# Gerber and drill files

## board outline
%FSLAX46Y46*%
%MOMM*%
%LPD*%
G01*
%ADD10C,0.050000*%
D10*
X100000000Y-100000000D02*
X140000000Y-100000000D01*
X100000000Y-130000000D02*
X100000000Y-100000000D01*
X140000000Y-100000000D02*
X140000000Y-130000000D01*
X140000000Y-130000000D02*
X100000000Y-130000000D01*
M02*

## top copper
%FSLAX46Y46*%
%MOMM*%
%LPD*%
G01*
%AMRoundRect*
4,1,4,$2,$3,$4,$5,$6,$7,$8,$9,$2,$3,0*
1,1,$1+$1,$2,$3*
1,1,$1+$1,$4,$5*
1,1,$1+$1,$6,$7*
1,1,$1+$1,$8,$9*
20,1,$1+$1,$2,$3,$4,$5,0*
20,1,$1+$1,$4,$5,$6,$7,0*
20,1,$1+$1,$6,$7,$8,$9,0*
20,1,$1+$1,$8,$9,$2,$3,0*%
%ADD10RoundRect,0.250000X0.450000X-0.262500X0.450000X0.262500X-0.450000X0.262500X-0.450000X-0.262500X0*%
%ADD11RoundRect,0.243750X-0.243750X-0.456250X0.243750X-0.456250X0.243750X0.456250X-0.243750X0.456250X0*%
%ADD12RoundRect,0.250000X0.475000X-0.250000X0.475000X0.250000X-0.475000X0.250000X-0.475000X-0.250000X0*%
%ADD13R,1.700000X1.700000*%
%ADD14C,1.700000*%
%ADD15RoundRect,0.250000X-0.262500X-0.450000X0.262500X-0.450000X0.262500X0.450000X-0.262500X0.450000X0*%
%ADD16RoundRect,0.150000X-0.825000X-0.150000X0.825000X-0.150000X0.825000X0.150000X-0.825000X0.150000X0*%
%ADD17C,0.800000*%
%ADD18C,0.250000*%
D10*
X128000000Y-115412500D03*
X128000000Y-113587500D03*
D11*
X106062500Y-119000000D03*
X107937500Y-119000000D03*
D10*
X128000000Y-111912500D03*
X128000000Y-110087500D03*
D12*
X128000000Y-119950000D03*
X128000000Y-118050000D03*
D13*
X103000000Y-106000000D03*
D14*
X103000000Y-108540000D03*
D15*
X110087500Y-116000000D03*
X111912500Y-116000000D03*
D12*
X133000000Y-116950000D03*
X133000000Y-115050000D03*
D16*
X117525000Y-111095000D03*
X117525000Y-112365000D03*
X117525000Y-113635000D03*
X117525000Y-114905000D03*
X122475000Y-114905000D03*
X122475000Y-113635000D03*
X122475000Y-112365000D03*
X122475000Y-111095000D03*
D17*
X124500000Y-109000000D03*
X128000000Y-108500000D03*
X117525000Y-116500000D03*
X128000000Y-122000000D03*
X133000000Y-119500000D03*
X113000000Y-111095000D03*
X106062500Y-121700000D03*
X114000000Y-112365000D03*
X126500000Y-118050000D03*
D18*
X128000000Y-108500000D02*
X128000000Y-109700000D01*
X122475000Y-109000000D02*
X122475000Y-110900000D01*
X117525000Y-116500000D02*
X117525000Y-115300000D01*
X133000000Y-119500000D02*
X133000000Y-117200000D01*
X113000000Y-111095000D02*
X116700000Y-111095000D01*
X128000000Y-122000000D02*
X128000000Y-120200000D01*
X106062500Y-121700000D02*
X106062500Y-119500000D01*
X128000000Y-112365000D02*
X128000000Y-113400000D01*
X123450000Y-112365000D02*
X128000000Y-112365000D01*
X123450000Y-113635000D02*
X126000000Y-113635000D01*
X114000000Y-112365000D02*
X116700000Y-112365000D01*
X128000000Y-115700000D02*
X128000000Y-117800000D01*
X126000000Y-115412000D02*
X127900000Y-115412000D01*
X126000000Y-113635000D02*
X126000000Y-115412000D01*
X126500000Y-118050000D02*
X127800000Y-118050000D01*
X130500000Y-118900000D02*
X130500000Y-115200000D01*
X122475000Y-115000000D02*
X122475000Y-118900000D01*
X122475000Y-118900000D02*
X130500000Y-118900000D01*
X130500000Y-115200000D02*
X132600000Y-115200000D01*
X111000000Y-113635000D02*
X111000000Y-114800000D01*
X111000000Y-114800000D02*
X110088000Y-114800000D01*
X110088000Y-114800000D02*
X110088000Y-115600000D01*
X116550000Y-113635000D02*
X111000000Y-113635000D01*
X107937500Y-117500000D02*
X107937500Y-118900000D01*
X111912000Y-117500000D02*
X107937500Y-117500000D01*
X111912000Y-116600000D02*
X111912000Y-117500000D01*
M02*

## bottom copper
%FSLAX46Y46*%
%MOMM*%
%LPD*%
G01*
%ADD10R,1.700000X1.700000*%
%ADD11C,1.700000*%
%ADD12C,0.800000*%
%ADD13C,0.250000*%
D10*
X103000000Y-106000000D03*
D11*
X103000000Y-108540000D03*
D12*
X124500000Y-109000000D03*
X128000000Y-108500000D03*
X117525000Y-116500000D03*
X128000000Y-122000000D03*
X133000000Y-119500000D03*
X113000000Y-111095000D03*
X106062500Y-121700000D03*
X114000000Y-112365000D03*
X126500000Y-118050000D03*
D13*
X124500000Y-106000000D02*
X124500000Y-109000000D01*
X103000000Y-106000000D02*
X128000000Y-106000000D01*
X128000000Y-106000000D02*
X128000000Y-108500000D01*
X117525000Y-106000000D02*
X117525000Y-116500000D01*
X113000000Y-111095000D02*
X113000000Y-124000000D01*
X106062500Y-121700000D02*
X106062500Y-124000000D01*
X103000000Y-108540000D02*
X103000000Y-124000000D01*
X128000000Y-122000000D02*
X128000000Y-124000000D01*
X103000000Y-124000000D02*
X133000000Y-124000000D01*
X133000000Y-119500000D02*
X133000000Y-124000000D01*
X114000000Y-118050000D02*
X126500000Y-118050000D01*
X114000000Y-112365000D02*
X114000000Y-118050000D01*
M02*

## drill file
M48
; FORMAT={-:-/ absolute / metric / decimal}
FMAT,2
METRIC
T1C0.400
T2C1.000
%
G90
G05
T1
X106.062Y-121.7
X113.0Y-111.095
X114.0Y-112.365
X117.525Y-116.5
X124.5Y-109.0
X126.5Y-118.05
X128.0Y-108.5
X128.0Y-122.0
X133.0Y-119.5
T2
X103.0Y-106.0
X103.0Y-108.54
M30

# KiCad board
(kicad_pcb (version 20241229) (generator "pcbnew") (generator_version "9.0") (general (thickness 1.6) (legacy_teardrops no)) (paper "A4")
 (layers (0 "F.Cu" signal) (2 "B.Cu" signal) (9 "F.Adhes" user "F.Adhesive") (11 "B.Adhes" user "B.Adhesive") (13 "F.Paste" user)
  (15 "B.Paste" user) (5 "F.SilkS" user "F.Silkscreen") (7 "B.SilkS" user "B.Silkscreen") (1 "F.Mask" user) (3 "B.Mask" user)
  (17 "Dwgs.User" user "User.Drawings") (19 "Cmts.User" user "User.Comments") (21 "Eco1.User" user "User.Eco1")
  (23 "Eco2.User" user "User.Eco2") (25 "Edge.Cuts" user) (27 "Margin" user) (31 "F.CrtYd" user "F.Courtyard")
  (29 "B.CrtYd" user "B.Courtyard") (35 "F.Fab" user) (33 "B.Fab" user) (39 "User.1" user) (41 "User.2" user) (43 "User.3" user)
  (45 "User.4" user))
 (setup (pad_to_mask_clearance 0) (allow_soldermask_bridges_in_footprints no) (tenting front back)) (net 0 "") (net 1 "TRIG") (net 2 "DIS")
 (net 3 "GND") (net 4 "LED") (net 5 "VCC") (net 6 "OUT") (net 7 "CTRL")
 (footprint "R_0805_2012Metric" (layer "F.Cu") (at 128 114.5 90)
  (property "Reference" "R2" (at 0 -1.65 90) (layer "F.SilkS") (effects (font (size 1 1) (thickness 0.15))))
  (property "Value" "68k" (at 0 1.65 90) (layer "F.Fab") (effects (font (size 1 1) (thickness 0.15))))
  (pad "1" smd roundrect (at -0.9125 0 90) (size 1.025 1.4) (layers "F.Cu" "F.Mask" "F.Paste") (roundrect_rratio 0.243902) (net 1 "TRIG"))
  (pad "2" smd roundrect (at 0.9125 0 90) (size 1.025 1.4) (layers "F.Cu" "F.Mask" "F.Paste") (roundrect_rratio 0.243902) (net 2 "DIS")))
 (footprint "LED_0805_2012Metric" (layer "F.Cu") (at 107 119)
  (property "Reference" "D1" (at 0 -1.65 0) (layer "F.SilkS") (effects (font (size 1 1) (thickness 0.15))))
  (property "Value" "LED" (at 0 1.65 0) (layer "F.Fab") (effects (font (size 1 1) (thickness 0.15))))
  (pad "1" smd roundrect (at -0.9375 0) (size 0.975 1.4) (layers "F.Cu" "F.Mask" "F.Paste") (roundrect_rratio 0.25) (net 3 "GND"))
  (pad "2" smd roundrect (at 0.9375 0) (size 0.975 1.4) (layers "F.Cu" "F.Mask" "F.Paste") (roundrect_rratio 0.25) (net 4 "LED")))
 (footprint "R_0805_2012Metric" (layer "F.Cu") (at 128 111 90)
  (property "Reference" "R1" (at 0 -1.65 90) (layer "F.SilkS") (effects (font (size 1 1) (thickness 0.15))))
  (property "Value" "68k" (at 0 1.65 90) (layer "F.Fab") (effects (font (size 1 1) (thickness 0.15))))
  (pad "1" smd roundrect (at -0.9125 0 90) (size 1.025 1.4) (layers "F.Cu" "F.Mask" "F.Paste") (roundrect_rratio 0.243902) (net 2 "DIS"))
  (pad "2" smd roundrect (at 0.9125 0 90) (size 1.025 1.4) (layers "F.Cu" "F.Mask" "F.Paste") (roundrect_rratio 0.243902) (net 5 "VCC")))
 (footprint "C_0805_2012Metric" (layer "F.Cu") (at 128 119 90)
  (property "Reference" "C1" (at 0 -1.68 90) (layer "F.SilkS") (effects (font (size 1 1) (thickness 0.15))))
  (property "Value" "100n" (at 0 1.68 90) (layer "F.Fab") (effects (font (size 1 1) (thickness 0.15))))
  (pad "1" smd roundrect (at -0.95 0 90) (size 1 1.45) (layers "F.Cu" "F.Mask" "F.Paste") (roundrect_rratio 0.25) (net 3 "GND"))
  (pad "2" smd roundrect (at 0.95 0 90) (size 1 1.45) (layers "F.Cu" "F.Mask" "F.Paste") (roundrect_rratio 0.25) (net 1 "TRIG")))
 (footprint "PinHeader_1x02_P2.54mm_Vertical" (layer "F.Cu") (at 103 106)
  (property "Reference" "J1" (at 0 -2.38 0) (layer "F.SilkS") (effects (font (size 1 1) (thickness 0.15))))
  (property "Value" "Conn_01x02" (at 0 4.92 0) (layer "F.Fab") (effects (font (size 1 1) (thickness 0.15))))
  (pad "1" thru_hole rect (at 0 0) (size 1.7 1.7) (drill 1) (layers "*.Cu" "*.Mask") (remove_unused_layers no) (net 5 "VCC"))
  (pad "2" thru_hole circle (at 0 2.54) (size 1.7 1.7) (drill 1) (layers "*.Cu" "*.Mask") (remove_unused_layers no) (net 3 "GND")))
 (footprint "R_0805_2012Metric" (layer "F.Cu") (at 111 116)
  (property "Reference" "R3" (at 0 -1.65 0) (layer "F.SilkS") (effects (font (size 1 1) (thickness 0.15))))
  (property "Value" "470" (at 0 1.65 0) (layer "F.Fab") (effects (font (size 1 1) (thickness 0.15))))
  (pad "1" smd roundrect (at -0.9125 0) (size 1.025 1.4) (layers "F.Cu" "F.Mask" "F.Paste") (roundrect_rratio 0.243902) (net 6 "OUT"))
  (pad "2" smd roundrect (at 0.9125 0) (size 1.025 1.4) (layers "F.Cu" "F.Mask" "F.Paste") (roundrect_rratio 0.243902) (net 4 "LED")))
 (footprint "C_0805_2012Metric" (layer "F.Cu") (at 133 116 90)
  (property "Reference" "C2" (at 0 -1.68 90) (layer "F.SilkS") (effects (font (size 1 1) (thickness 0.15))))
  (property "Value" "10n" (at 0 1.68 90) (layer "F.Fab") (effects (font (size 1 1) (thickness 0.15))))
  (pad "1" smd roundrect (at -0.95 0 90) (size 1 1.45) (layers "F.Cu" "F.Mask" "F.Paste") (roundrect_rratio 0.25) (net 3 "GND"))
  (pad "2" smd roundrect (at 0.95 0 90) (size 1 1.45) (layers "F.Cu" "F.Mask" "F.Paste") (roundrect_rratio 0.25) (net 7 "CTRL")))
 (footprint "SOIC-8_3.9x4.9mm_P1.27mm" (layer "F.Cu") (at 120 113)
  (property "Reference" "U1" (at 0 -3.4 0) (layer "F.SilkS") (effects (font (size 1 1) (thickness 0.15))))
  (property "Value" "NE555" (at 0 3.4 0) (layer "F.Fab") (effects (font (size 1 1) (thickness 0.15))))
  (pad "1" smd roundrect (at -2.475 -1.905) (size 1.95 0.6) (layers "F.Cu" "F.Mask" "F.Paste") (roundrect_rratio 0.25) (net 3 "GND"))
  (pad "2" smd roundrect (at -2.475 -0.635) (size 1.95 0.6) (layers "F.Cu" "F.Mask" "F.Paste") (roundrect_rratio 0.25) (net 1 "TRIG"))
  (pad "3" smd roundrect (at -2.475 0.635) (size 1.95 0.6) (layers "F.Cu" "F.Mask" "F.Paste") (roundrect_rratio 0.25) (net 6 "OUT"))
  (pad "4" smd roundrect (at -2.475 1.905) (size 1.95 0.6) (layers "F.Cu" "F.Mask" "F.Paste") (roundrect_rratio 0.25) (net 5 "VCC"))
  (pad "5" smd roundrect (at 2.475 1.905) (size 1.95 0.6) (layers "F.Cu" "F.Mask" "F.Paste") (roundrect_rratio 0.25) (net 7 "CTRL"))
  (pad "6" smd roundrect (at 2.475 0.635) (size 1.95 0.6) (layers "F.Cu" "F.Mask" "F.Paste") (roundrect_rratio 0.25) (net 1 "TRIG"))
  (pad "7" smd roundrect (at 2.475 -0.635) (size 1.95 0.6) (layers "F.Cu" "F.Mask" "F.Paste") (roundrect_rratio 0.25) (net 2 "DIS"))
  (pad "8" smd roundrect (at 2.475 -1.905) (size 1.95 0.6) (layers "F.Cu" "F.Mask" "F.Paste") (roundrect_rratio 0.25) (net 5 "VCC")))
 (gr_line (start 100 100) (end 140 100) (stroke (width 0.05) (type default)) (layer "Edge.Cuts"))
 (gr_line (start 100 130) (end 100 100) (stroke (width 0.05) (type default)) (layer "Edge.Cuts"))
 (gr_line (start 140 100) (end 140 130) (stroke (width 0.05) (type default)) (layer "Edge.Cuts"))
 (gr_line (start 140 130) (end 100 130) (stroke (width 0.05) (type default)) (layer "Edge.Cuts"))
 (segment (start 128 108.5) (end 128 109.7) (width 0.25) (layer "F.Cu") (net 5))
 (segment (start 122.475 109) (end 122.475 110.9) (width 0.25) (layer "F.Cu") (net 5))
 (segment (start 117.525 116.5) (end 117.525 115.3) (width 0.25) (layer "F.Cu") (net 5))
 (via (at 124.5 109) (size 0.8) (drill 0.4) (layers "F.Cu" "B.Cu") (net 5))
 (via (at 128 108.5) (size 0.8) (drill 0.4) (layers "F.Cu" "B.Cu") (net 5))
 (via (at 117.525 116.5) (size 0.8) (drill 0.4) (layers "F.Cu" "B.Cu") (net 5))
 (segment (start 124.5 106) (end 124.5 109) (width 0.25) (layer "B.Cu") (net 5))
 (segment (start 103 106) (end 128 106) (width 0.25) (layer "B.Cu") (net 5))
 (segment (start 128 106) (end 128 108.5) (width 0.25) (layer "B.Cu") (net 5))
 (segment (start 117.525 106) (end 117.525 116.5) (width 0.25) (layer "B.Cu") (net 5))
 (segment (start 133 119.5) (end 133 117.2) (width 0.25) (layer "F.Cu") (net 3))
 (segment (start 113 111.095) (end 116.7 111.095) (width 0.25) (layer "F.Cu") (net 3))
 (segment (start 128 122) (end 128 120.2) (width 0.25) (layer "F.Cu") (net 3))
 (segment (start 106.0625 121.7) (end 106.0625 119.5) (width 0.25) (layer "F.Cu") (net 3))
 (via (at 128 122) (size 0.8) (drill 0.4) (layers "F.Cu" "B.Cu") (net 3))
 (via (at 133 119.5) (size 0.8) (drill 0.4) (layers "F.Cu" "B.Cu") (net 3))
 (via (at 113 111.095) (size 0.8) (drill 0.4) (layers "F.Cu" "B.Cu") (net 3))
 (via (at 106.0625 121.7) (size 0.8) (drill 0.4) (layers "F.Cu" "B.Cu") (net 3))
 (segment (start 113 111.095) (end 113 124) (width 0.25) (layer "B.Cu") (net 3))
 (segment (start 106.0625 121.7) (end 106.0625 124) (width 0.25) (layer "B.Cu") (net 3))
 (segment (start 103 108.54) (end 103 124) (width 0.25) (layer "B.Cu") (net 3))
 (segment (start 128 122) (end 128 124) (width 0.25) (layer "B.Cu") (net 3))
 (segment (start 103 124) (end 133 124) (width 0.25) (layer "B.Cu") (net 3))
 (segment (start 133 119.5) (end 133 124) (width 0.25) (layer "B.Cu") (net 3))
 (segment (start 128 112.365) (end 128 113.4) (width 0.25) (layer "F.Cu") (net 2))
 (segment (start 123.45 112.365) (end 128 112.365) (width 0.25) (layer "F.Cu") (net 2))
 (segment (start 123.45 113.635) (end 126 113.635) (width 0.25) (layer "F.Cu") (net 1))
 (segment (start 114 112.365) (end 116.7 112.365) (width 0.25) (layer "F.Cu") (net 1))
 (segment (start 128 115.7) (end 128 117.8) (width 0.25) (layer "F.Cu") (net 1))
 (segment (start 126 115.412) (end 127.9 115.412) (width 0.25) (layer "F.Cu") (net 1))
 (segment (start 126 113.635) (end 126 115.412) (width 0.25) (layer "F.Cu") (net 1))
 (segment (start 126.5 118.05) (end 127.8 118.05) (width 0.25) (layer "F.Cu") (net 1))
 (via (at 114 112.365) (size 0.8) (drill 0.4) (layers "F.Cu" "B.Cu") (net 1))
 (via (at 126.5 118.05) (size 0.8) (drill 0.4) (layers "F.Cu" "B.Cu") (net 1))
 (segment (start 114 118.05) (end 126.5 118.05) (width 0.25) (layer "B.Cu") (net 1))
 (segment (start 114 112.365) (end 114 118.05) (width 0.25) (layer "B.Cu") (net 1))
 (segment (start 130.5 118.9) (end 130.5 115.2) (width 0.25) (layer "F.Cu") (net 7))
 (segment (start 122.475 115) (end 122.475 118.9) (width 0.25) (layer "F.Cu") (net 7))
 (segment (start 122.475 118.9) (end 130.5 118.9) (width 0.25) (layer "F.Cu") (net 7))
 (segment (start 130.5 115.2) (end 132.6 115.2) (width 0.25) (layer "F.Cu") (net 7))
 (segment (start 111 113.635) (end 111 114.8) (width 0.25) (layer "F.Cu") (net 6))
 (segment (start 111 114.8) (end 110.088 114.8) (width 0.25) (layer "F.Cu") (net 6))
 (segment (start 110.088 114.8) (end 110.088 115.6) (width 0.25) (layer "F.Cu") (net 6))
 (segment (start 116.55 113.635) (end 111 113.635) (width 0.25) (layer "F.Cu") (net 6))
 (segment (start 107.9375 117.5) (end 107.9375 118.9) (width 0.25) (layer "F.Cu") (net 4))
 (segment (start 111.912 117.5) (end 107.9375 117.5) (width 0.25) (layer "F.Cu") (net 4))
 (segment (start 111.912 116.6) (end 111.912 117.5) (width 0.25) (layer "F.Cu") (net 4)))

